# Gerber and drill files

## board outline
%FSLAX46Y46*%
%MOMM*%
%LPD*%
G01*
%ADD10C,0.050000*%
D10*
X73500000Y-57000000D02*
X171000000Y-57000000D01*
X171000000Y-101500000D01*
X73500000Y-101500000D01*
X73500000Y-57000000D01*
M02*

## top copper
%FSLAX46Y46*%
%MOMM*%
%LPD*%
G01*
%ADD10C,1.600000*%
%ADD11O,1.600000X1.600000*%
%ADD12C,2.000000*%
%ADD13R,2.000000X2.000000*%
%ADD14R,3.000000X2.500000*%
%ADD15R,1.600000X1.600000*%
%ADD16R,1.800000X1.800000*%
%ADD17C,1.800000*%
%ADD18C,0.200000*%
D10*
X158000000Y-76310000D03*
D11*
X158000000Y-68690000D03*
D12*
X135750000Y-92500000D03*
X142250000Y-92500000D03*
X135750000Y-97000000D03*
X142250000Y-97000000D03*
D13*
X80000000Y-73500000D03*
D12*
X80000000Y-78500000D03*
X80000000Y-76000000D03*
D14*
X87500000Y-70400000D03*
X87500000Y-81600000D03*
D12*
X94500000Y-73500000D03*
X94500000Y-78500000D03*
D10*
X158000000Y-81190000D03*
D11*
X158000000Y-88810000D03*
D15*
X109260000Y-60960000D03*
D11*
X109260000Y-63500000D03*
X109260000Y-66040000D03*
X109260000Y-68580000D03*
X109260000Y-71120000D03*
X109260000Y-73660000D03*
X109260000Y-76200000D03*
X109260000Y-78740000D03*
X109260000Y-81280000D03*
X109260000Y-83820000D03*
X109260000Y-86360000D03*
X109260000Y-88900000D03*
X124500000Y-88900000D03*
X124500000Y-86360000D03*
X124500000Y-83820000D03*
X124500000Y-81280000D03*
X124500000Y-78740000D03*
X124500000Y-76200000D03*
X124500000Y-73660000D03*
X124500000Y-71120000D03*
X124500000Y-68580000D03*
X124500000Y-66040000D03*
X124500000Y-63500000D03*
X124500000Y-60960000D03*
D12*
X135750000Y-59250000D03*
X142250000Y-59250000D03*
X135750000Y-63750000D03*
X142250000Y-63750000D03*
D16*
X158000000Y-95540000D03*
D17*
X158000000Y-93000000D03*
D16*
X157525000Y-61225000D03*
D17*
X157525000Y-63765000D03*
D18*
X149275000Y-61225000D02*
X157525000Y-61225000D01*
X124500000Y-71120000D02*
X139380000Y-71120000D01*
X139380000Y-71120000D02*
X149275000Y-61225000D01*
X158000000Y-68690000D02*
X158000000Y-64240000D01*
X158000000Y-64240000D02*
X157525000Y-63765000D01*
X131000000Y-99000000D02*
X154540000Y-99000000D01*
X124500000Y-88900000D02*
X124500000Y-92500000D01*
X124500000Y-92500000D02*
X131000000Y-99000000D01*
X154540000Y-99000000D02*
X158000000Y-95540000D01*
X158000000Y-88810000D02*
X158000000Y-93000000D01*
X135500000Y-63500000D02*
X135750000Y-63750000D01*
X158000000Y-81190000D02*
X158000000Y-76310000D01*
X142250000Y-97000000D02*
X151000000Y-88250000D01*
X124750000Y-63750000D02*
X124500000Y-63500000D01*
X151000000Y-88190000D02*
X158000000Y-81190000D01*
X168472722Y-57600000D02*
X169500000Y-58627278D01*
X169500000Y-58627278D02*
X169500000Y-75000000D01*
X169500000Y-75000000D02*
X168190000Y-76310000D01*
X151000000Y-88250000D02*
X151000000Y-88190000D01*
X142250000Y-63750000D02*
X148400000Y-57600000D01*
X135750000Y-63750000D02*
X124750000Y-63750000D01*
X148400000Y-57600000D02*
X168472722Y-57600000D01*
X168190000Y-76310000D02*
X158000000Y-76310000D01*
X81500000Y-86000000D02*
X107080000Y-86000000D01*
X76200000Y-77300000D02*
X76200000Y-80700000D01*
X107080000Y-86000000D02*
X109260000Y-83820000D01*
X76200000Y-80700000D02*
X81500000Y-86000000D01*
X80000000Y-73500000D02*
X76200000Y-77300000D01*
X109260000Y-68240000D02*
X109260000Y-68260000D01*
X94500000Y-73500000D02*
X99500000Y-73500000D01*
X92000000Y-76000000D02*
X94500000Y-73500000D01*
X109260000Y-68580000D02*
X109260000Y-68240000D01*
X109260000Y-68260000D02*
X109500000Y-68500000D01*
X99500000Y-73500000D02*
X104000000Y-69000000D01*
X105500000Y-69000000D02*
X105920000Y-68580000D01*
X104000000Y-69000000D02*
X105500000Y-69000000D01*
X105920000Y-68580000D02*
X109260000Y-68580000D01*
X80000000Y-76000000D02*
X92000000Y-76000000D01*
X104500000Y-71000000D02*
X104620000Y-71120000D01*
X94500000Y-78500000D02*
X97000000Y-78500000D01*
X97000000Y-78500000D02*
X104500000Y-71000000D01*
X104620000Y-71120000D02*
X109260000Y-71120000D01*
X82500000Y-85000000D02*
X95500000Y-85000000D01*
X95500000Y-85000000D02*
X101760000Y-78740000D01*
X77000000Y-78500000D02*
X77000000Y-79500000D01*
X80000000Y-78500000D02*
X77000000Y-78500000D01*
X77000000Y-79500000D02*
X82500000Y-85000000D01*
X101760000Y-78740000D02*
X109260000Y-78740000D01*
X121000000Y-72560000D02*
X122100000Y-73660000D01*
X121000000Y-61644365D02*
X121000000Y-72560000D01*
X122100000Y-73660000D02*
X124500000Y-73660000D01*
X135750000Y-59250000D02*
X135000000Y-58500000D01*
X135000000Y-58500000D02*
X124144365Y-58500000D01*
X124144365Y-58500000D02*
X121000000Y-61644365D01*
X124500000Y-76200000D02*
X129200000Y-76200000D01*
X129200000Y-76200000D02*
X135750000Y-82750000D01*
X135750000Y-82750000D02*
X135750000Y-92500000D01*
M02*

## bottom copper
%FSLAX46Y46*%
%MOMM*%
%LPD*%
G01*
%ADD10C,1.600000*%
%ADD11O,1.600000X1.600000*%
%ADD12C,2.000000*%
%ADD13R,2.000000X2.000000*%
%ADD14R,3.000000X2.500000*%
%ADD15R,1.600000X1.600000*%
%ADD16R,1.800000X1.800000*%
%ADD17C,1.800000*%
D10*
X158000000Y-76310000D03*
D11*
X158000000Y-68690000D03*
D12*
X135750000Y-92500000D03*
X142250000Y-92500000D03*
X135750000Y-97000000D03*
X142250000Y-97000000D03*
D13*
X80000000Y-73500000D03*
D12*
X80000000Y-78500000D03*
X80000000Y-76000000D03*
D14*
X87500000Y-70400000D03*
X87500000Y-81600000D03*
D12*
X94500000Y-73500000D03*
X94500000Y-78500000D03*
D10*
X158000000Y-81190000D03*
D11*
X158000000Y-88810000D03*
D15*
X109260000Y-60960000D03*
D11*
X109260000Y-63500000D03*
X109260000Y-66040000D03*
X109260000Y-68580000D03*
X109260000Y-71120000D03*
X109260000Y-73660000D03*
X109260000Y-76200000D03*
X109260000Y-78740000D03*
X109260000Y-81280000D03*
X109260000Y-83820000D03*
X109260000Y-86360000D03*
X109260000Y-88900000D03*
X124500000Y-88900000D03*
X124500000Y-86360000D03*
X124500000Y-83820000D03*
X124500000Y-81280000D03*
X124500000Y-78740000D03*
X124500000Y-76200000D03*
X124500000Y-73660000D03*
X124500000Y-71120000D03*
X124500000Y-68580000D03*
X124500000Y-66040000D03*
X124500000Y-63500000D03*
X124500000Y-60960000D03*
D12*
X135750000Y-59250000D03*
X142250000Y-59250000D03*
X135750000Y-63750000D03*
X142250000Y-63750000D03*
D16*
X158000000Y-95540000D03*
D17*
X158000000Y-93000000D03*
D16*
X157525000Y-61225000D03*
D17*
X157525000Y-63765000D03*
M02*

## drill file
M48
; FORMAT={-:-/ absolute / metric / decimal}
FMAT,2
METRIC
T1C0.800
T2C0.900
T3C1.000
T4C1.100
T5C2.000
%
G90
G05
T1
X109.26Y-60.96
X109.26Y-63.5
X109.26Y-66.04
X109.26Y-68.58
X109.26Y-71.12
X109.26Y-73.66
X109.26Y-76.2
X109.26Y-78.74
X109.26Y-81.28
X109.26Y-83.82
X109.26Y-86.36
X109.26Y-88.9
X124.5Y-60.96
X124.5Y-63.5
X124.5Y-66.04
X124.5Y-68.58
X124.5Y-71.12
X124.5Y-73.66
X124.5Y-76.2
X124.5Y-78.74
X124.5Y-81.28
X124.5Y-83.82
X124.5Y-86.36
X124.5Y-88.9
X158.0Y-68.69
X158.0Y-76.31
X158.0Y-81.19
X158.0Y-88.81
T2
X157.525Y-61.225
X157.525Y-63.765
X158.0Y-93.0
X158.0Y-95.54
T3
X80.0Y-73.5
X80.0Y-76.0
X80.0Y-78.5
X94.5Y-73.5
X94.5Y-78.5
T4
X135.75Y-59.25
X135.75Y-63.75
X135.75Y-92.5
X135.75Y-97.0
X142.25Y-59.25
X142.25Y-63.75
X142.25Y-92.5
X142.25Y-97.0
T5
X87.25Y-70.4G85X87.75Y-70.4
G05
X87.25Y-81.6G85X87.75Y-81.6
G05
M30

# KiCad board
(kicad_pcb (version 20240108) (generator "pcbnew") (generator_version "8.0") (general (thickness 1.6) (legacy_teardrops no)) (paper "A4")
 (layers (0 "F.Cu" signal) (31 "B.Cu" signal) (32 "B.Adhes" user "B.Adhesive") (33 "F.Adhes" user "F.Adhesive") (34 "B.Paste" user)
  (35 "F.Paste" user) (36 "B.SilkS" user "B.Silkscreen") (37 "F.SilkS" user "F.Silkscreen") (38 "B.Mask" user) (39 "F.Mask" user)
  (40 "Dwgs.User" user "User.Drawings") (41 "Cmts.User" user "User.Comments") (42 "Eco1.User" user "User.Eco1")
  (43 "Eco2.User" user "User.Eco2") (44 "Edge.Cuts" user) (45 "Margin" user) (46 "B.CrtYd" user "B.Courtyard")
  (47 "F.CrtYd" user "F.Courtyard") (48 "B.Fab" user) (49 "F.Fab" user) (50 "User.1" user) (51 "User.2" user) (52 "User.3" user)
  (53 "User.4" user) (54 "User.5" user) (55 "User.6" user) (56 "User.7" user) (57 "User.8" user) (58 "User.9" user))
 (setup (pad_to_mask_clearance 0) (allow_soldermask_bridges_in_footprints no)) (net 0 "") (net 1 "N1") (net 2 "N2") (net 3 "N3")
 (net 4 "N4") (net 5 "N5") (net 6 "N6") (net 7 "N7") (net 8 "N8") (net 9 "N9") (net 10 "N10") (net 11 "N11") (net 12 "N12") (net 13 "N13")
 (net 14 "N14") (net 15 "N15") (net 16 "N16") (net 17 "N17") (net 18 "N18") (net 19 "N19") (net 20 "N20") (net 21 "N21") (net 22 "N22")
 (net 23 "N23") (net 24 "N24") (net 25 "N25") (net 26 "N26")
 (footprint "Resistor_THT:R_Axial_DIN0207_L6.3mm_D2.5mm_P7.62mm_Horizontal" (layer "F.Cu") (at 158 76.31 90)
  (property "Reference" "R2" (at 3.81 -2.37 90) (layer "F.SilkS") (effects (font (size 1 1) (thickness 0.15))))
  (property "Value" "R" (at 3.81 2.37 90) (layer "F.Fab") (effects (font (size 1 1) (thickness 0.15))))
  (pad "1" thru_hole circle (at 0 0 90) (size 1.6 1.6) (drill 0.8) (layers "*.Cu" "*.Mask") (remove_unused_layers no) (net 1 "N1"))
  (pad "2" thru_hole oval (at 7.62 0 90) (size 1.6 1.6) (drill 0.8) (layers "*.Cu" "*.Mask") (remove_unused_layers no) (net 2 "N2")))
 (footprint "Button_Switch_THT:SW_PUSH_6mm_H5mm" (layer "F.Cu") (at 135.75 92.5)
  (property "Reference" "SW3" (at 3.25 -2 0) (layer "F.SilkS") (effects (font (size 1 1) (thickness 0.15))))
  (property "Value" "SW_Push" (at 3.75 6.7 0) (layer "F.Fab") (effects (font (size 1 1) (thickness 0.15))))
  (pad "1" thru_hole circle (at 0 0 90) (size 2 2) (drill 1.1) (layers "*.Cu" "*.Mask") (remove_unused_layers no) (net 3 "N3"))
  (pad "1" thru_hole circle (at 6.5 0 90) (size 2 2) (drill 1.1) (layers "*.Cu" "*.Mask") (remove_unused_layers no) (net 3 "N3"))
  (pad "2" thru_hole circle (at 0 4.5 90) (size 2 2) (drill 1.1) (layers "*.Cu" "*.Mask") (remove_unused_layers no) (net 1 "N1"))
  (pad "2" thru_hole circle (at 6.5 4.5 90) (size 2 2) (drill 1.1) (layers "*.Cu" "*.Mask") (remove_unused_layers no) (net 1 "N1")))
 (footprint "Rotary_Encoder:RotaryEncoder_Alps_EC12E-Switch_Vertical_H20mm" (layer "F.Cu") (at 80 73.5)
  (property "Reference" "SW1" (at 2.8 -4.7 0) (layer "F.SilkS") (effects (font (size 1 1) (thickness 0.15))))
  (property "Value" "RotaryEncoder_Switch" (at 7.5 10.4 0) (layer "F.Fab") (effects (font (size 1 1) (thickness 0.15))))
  (pad "A" thru_hole rect (at 0 0) (size 2 2) (drill 1) (layers "*.Cu" "*.Mask") (remove_unused_layers no) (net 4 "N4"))
  (pad "B" thru_hole circle (at 0 5) (size 2 2) (drill 1) (layers "*.Cu" "*.Mask") (remove_unused_layers no) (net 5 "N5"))
  (pad "C" thru_hole circle (at 0 2.5) (size 2 2) (drill 1) (layers "*.Cu" "*.Mask") (remove_unused_layers no) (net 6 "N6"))
  (pad "MP" thru_hole rect (at 7.5 -3.1) (size 3 2.5) (drill oval 2.5 2) (layers "*.Cu" "*.Mask") (remove_unused_layers no))
  (pad "MP" thru_hole rect (at 7.5 8.1) (size 3 2.5) (drill oval 2.5 2) (layers "*.Cu" "*.Mask") (remove_unused_layers no))
  (pad "S1" thru_hole circle (at 14.5 0) (size 2 2) (drill 1) (layers "*.Cu" "*.Mask") (remove_unused_layers no) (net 6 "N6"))
  (pad "S2" thru_hole circle (at 14.5 5) (size 2 2) (drill 1) (layers "*.Cu" "*.Mask") (remove_unused_layers no) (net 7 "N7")))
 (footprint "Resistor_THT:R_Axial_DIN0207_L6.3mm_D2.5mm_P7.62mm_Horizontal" (layer "F.Cu") (at 158 81.19 -90)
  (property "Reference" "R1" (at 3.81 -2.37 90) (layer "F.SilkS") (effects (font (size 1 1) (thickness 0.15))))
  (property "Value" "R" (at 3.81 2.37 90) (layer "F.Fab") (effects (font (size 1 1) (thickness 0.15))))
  (pad "1" thru_hole circle (at 0 0 270) (size 1.6 1.6) (drill 0.8) (layers "*.Cu" "*.Mask") (remove_unused_layers no) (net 1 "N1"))
  (pad "2" thru_hole oval (at 7.62 0 270) (size 1.6 1.6) (drill 0.8) (layers "*.Cu" "*.Mask") (remove_unused_layers no) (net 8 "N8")))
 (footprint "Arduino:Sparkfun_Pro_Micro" (layer "F.Cu") (at 124.5 88.9 180)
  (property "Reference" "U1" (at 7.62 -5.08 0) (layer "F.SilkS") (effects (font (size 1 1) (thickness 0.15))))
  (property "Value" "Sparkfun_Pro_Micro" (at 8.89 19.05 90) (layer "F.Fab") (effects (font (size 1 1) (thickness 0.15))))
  (pad "1" thru_hole rect (at 15.24 27.94 180) (size 1.6 1.6) (drill 0.8) (layers "*.Cu" "*.Mask") (remove_unused_layers no) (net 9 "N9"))
  (pad "2" thru_hole oval (at 15.24 25.4 180) (size 1.6 1.6) (drill 0.8) (layers "*.Cu" "*.Mask") (remove_unused_layers no) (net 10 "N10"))
  (pad "3" thru_hole oval (at 15.24 22.86 180) (size 1.6 1.6) (drill 0.8) (layers "*.Cu" "*.Mask") (remove_unused_layers no) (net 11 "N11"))
  (pad "4" thru_hole oval (at 15.24 20.32 180) (size 1.6 1.6) (drill 0.8) (layers "*.Cu" "*.Mask") (remove_unused_layers no) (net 6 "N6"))
  (pad "5" thru_hole oval (at 15.24 17.78 180) (size 1.6 1.6) (drill 0.8) (layers "*.Cu" "*.Mask") (remove_unused_layers no) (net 7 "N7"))
  (pad "6" thru_hole oval (at 15.24 15.24 180) (size 1.6 1.6) (drill 0.8) (layers "*.Cu" "*.Mask") (remove_unused_layers no) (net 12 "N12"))
  (pad "7" thru_hole oval (at 15.24 12.7 180) (size 1.6 1.6) (drill 0.8) (layers "*.Cu" "*.Mask") (remove_unused_layers no) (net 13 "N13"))
  (pad "8" thru_hole oval (at 15.24 10.16 180) (size 1.6 1.6) (drill 0.8) (layers "*.Cu" "*.Mask") (remove_unused_layers no) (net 5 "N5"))
  (pad "9" thru_hole oval (at 15.24 7.62 180) (size 1.6 1.6) (drill 0.8) (layers "*.Cu" "*.Mask") (remove_unused_layers no) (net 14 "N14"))
  (pad "10" thru_hole oval (at 15.24 5.08 180) (size 1.6 1.6) (drill 0.8) (layers "*.Cu" "*.Mask") (remove_unused_layers no) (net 4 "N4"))
  (pad "11" thru_hole oval (at 15.24 2.54 180) (size 1.6 1.6) (drill 0.8) (layers "*.Cu" "*.Mask") (remove_unused_layers no) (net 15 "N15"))
  (pad "12" thru_hole oval (at 15.24 0 180) (size 1.6 1.6) (drill 0.8) (layers "*.Cu" "*.Mask") (remove_unused_layers no) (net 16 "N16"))
  (pad "13" thru_hole oval (at 0 0 180) (size 1.6 1.6) (drill 0.8) (layers "*.Cu" "*.Mask") (remove_unused_layers no) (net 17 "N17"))
  (pad "14" thru_hole oval (at 0 2.54 180) (size 1.6 1.6) (drill 0.8) (layers "*.Cu" "*.Mask") (remove_unused_layers no) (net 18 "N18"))
  (pad "15" thru_hole oval (at 0 5.08 180) (size 1.6 1.6) (drill 0.8) (layers "*.Cu" "*.Mask") (remove_unused_layers no) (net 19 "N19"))
  (pad "16" thru_hole oval (at 0 7.62 180) (size 1.6 1.6) (drill 0.8) (layers "*.Cu" "*.Mask") (remove_unused_layers no) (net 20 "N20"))
  (pad "17" thru_hole oval (at 0 10.16 180) (size 1.6 1.6) (drill 0.8) (layers "*.Cu" "*.Mask") (remove_unused_layers no) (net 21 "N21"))
  (pad "18" thru_hole oval (at 0 12.7 180) (size 1.6 1.6) (drill 0.8) (layers "*.Cu" "*.Mask") (remove_unused_layers no) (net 3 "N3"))
  (pad "19" thru_hole oval (at 0 15.24 180) (size 1.6 1.6) (drill 0.8) (layers "*.Cu" "*.Mask") (remove_unused_layers no) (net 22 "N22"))
  (pad "20" thru_hole oval (at 0 17.78 180) (size 1.6 1.6) (drill 0.8) (layers "*.Cu" "*.Mask") (remove_unused_layers no) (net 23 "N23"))
  (pad "21" thru_hole oval (at 0 20.32 180) (size 1.6 1.6) (drill 0.8) (layers "*.Cu" "*.Mask") (remove_unused_layers no) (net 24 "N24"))
  (pad "22" thru_hole oval (at 0 22.86 180) (size 1.6 1.6) (drill 0.8) (layers "*.Cu" "*.Mask") (remove_unused_layers no) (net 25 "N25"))
  (pad "23" thru_hole oval (at 0 25.4 180) (size 1.6 1.6) (drill 0.8) (layers "*.Cu" "*.Mask") (remove_unused_layers no) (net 1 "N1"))
  (pad "24" thru_hole oval (at 0 27.94 180) (size 1.6 1.6) (drill 0.8) (layers "*.Cu" "*.Mask") (remove_unused_layers no) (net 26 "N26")))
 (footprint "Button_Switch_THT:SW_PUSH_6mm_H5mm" (layer "F.Cu") (at 135.75 59.25)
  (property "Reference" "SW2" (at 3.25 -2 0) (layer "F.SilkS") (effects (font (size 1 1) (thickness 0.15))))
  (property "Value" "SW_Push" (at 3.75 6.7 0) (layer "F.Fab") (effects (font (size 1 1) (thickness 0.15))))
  (pad "1" thru_hole circle (at 0 0 90) (size 2 2) (drill 1.1) (layers "*.Cu" "*.Mask") (remove_unused_layers no) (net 22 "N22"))
  (pad "1" thru_hole circle (at 6.5 0 90) (size 2 2) (drill 1.1) (layers "*.Cu" "*.Mask") (remove_unused_layers no) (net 22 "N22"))
  (pad "2" thru_hole circle (at 0 4.5 90) (size 2 2) (drill 1.1) (layers "*.Cu" "*.Mask") (remove_unused_layers no) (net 1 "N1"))
  (pad "2" thru_hole circle (at 6.5 4.5 90) (size 2 2) (drill 1.1) (layers "*.Cu" "*.Mask") (remove_unused_layers no) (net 1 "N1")))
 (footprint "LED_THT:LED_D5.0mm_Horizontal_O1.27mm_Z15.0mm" (layer "F.Cu") (at 158 95.54 90)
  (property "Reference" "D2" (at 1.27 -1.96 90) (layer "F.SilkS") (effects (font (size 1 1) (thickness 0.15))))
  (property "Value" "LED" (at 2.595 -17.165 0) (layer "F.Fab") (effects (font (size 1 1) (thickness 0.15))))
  (pad "1" thru_hole rect (at 0 0 90) (size 1.8 1.8) (drill 0.9) (layers "*.Cu" "*.Mask") (remove_unused_layers no) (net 17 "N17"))
  (pad "2" thru_hole circle (at 2.54 0 90) (size 1.8 1.8) (drill 0.9) (layers "*.Cu" "*.Mask") (remove_unused_layers no) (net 8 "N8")))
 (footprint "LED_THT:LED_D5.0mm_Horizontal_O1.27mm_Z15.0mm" (layer "B.Cu") (at 157.525 61.225 -90)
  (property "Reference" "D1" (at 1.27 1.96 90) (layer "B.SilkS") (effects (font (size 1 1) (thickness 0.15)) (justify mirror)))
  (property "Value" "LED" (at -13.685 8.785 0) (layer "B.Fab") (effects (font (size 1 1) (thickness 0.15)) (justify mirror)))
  (pad "1" thru_hole rect (at 0 0 270) (size 1.8 1.8) (drill 0.9) (layers "*.Cu" "*.Mask") (remove_unused_layers no) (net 23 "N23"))
  (pad "2" thru_hole circle (at 2.54 0 270) (size 1.8 1.8) (drill 0.9) (layers "*.Cu" "*.Mask") (remove_unused_layers no) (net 2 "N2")))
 (gr_rect (start 73.5 57) (end 171 101.5) (stroke (width 0.05) (type default)) (fill none) (layer "Edge.Cuts"))
 (segment (start 149.275 61.225) (end 157.525 61.225) (width 0.2) (layer "F.Cu") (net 23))
 (segment (start 124.5 71.12) (end 139.38 71.12) (width 0.2) (layer "F.Cu") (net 23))
 (segment (start 139.38 71.12) (end 149.275 61.225) (width 0.2) (layer "F.Cu") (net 23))
 (segment (start 158 68.69) (end 158 64.24) (width 0.2) (layer "F.Cu") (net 2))
 (segment (start 158 64.24) (end 157.525 63.765) (width 0.2) (layer "F.Cu") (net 2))
 (segment (start 131 99) (end 154.54 99) (width 0.2) (layer "F.Cu") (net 17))
 (segment (start 124.5 88.9) (end 124.5 92.5) (width 0.2) (layer "F.Cu") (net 17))
 (segment (start 124.5 92.5) (end 131 99) (width 0.2) (layer "F.Cu") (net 17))
 (segment (start 154.54 99) (end 158 95.54) (width 0.2) (layer "F.Cu") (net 17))
 (segment (start 158 88.81) (end 158 93) (width 0.2) (layer "F.Cu") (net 8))
 (segment (start 135.5 63.5) (end 135.75 63.75) (width 0.2) (layer "F.Cu") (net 1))
 (segment (start 158 81.19) (end 158 76.31) (width 0.2) (layer "F.Cu") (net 1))
 (segment (start 142.25 97) (end 151 88.25) (width 0.2) (layer "F.Cu") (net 1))
 (segment (start 124.75 63.75) (end 124.5 63.5) (width 0.2) (layer "F.Cu") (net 1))
 (segment (start 151 88.19) (end 158 81.19) (width 0.2) (layer "F.Cu") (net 1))
 (segment (start 168.472722 57.6) (end 169.5 58.627278) (width 0.2) (layer "F.Cu") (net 1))
 (segment (start 169.5 58.627278) (end 169.5 75) (width 0.2) (layer "F.Cu") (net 1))
 (segment (start 169.5 75) (end 168.19 76.31) (width 0.2) (layer "F.Cu") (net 1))
 (segment (start 151 88.25) (end 151 88.19) (width 0.2) (layer "F.Cu") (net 1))
 (segment (start 142.25 63.75) (end 148.4 57.6) (width 0.2) (layer "F.Cu") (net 1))
 (segment (start 135.75 63.75) (end 124.75 63.75) (width 0.2) (layer "F.Cu") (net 1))
 (segment (start 148.4 57.6) (end 168.472722 57.6) (width 0.2) (layer "F.Cu") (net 1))
 (segment (start 168.19 76.31) (end 158 76.31) (width 0.2) (layer "F.Cu") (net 1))
 (segment (start 81.5 86) (end 107.08 86) (width 0.2) (layer "F.Cu") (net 4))
 (segment (start 76.2 77.3) (end 76.2 80.7) (width 0.2) (layer "F.Cu") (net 4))
 (segment (start 107.08 86) (end 109.26 83.82) (width 0.2) (layer "F.Cu") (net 4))
 (segment (start 76.2 80.7) (end 81.5 86) (width 0.2) (layer "F.Cu") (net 4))
 (segment (start 80 73.5) (end 76.2 77.3) (width 0.2) (layer "F.Cu") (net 4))
 (segment (start 109.26 68.24) (end 109.26 68.26) (width 0.2) (layer "F.Cu") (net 6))
 (segment (start 94.5 73.5) (end 99.5 73.5) (width 0.2) (layer "F.Cu") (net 6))
 (segment (start 92 76) (end 94.5 73.5) (width 0.2) (layer "F.Cu") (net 6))
 (segment (start 109.26 68.58) (end 109.26 68.24) (width 0.2) (layer "F.Cu") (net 6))
 (segment (start 109.26 68.26) (end 109.5 68.5) (width 0.2) (layer "F.Cu") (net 6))
 (segment (start 99.5 73.5) (end 104 69) (width 0.2) (layer "F.Cu") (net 6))
 (segment (start 105.5 69) (end 105.92 68.58) (width 0.2) (layer "F.Cu") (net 6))
 (segment (start 104 69) (end 105.5 69) (width 0.2) (layer "F.Cu") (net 6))
 (segment (start 105.92 68.58) (end 109.26 68.58) (width 0.2) (layer "F.Cu") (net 6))
 (segment (start 80 76) (end 92 76) (width 0.2) (layer "F.Cu") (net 6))
 (segment (start 104.5 71) (end 104.62 71.12) (width 0.2) (layer "F.Cu") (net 7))
 (segment (start 94.5 78.5) (end 97 78.5) (width 0.2) (layer "F.Cu") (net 7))
 (segment (start 97 78.5) (end 104.5 71) (width 0.2) (layer "F.Cu") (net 7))
 (segment (start 104.62 71.12) (end 109.26 71.12) (width 0.2) (layer "F.Cu") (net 7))
 (segment (start 82.5 85) (end 95.5 85) (width 0.2) (layer "F.Cu") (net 5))
 (segment (start 95.5 85) (end 101.76 78.74) (width 0.2) (layer "F.Cu") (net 5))
 (segment (start 77 78.5) (end 77 79.5) (width 0.2) (layer "F.Cu") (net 5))
 (segment (start 80 78.5) (end 77 78.5) (width 0.2) (layer "F.Cu") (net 5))
 (segment (start 77 79.5) (end 82.5 85) (width 0.2) (layer "F.Cu") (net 5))
 (segment (start 101.76 78.74) (end 109.26 78.74) (width 0.2) (layer "F.Cu") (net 5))
 (segment (start 121 72.56) (end 122.1 73.66) (width 0.2) (layer "F.Cu") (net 22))
 (segment (start 121 61.644365) (end 121 72.56) (width 0.2) (layer "F.Cu") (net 22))
 (segment (start 122.1 73.66) (end 124.5 73.66) (width 0.2) (layer "F.Cu") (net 22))
 (segment (start 135.75 59.25) (end 135 58.5) (width 0.2) (layer "F.Cu") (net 22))
 (segment (start 135 58.5) (end 124.144365 58.5) (width 0.2) (layer "F.Cu") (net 22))
 (segment (start 124.144365 58.5) (end 121 61.644365) (width 0.2) (layer "F.Cu") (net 22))
 (segment (start 124.5 76.2) (end 129.2 76.2) (width 0.2) (layer "F.Cu") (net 3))
 (segment (start 129.2 76.2) (end 135.75 82.75) (width 0.2) (layer "F.Cu") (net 3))
 (segment (start 135.75 82.75) (end 135.75 92.5) (width 0.2) (layer "F.Cu") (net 3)))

